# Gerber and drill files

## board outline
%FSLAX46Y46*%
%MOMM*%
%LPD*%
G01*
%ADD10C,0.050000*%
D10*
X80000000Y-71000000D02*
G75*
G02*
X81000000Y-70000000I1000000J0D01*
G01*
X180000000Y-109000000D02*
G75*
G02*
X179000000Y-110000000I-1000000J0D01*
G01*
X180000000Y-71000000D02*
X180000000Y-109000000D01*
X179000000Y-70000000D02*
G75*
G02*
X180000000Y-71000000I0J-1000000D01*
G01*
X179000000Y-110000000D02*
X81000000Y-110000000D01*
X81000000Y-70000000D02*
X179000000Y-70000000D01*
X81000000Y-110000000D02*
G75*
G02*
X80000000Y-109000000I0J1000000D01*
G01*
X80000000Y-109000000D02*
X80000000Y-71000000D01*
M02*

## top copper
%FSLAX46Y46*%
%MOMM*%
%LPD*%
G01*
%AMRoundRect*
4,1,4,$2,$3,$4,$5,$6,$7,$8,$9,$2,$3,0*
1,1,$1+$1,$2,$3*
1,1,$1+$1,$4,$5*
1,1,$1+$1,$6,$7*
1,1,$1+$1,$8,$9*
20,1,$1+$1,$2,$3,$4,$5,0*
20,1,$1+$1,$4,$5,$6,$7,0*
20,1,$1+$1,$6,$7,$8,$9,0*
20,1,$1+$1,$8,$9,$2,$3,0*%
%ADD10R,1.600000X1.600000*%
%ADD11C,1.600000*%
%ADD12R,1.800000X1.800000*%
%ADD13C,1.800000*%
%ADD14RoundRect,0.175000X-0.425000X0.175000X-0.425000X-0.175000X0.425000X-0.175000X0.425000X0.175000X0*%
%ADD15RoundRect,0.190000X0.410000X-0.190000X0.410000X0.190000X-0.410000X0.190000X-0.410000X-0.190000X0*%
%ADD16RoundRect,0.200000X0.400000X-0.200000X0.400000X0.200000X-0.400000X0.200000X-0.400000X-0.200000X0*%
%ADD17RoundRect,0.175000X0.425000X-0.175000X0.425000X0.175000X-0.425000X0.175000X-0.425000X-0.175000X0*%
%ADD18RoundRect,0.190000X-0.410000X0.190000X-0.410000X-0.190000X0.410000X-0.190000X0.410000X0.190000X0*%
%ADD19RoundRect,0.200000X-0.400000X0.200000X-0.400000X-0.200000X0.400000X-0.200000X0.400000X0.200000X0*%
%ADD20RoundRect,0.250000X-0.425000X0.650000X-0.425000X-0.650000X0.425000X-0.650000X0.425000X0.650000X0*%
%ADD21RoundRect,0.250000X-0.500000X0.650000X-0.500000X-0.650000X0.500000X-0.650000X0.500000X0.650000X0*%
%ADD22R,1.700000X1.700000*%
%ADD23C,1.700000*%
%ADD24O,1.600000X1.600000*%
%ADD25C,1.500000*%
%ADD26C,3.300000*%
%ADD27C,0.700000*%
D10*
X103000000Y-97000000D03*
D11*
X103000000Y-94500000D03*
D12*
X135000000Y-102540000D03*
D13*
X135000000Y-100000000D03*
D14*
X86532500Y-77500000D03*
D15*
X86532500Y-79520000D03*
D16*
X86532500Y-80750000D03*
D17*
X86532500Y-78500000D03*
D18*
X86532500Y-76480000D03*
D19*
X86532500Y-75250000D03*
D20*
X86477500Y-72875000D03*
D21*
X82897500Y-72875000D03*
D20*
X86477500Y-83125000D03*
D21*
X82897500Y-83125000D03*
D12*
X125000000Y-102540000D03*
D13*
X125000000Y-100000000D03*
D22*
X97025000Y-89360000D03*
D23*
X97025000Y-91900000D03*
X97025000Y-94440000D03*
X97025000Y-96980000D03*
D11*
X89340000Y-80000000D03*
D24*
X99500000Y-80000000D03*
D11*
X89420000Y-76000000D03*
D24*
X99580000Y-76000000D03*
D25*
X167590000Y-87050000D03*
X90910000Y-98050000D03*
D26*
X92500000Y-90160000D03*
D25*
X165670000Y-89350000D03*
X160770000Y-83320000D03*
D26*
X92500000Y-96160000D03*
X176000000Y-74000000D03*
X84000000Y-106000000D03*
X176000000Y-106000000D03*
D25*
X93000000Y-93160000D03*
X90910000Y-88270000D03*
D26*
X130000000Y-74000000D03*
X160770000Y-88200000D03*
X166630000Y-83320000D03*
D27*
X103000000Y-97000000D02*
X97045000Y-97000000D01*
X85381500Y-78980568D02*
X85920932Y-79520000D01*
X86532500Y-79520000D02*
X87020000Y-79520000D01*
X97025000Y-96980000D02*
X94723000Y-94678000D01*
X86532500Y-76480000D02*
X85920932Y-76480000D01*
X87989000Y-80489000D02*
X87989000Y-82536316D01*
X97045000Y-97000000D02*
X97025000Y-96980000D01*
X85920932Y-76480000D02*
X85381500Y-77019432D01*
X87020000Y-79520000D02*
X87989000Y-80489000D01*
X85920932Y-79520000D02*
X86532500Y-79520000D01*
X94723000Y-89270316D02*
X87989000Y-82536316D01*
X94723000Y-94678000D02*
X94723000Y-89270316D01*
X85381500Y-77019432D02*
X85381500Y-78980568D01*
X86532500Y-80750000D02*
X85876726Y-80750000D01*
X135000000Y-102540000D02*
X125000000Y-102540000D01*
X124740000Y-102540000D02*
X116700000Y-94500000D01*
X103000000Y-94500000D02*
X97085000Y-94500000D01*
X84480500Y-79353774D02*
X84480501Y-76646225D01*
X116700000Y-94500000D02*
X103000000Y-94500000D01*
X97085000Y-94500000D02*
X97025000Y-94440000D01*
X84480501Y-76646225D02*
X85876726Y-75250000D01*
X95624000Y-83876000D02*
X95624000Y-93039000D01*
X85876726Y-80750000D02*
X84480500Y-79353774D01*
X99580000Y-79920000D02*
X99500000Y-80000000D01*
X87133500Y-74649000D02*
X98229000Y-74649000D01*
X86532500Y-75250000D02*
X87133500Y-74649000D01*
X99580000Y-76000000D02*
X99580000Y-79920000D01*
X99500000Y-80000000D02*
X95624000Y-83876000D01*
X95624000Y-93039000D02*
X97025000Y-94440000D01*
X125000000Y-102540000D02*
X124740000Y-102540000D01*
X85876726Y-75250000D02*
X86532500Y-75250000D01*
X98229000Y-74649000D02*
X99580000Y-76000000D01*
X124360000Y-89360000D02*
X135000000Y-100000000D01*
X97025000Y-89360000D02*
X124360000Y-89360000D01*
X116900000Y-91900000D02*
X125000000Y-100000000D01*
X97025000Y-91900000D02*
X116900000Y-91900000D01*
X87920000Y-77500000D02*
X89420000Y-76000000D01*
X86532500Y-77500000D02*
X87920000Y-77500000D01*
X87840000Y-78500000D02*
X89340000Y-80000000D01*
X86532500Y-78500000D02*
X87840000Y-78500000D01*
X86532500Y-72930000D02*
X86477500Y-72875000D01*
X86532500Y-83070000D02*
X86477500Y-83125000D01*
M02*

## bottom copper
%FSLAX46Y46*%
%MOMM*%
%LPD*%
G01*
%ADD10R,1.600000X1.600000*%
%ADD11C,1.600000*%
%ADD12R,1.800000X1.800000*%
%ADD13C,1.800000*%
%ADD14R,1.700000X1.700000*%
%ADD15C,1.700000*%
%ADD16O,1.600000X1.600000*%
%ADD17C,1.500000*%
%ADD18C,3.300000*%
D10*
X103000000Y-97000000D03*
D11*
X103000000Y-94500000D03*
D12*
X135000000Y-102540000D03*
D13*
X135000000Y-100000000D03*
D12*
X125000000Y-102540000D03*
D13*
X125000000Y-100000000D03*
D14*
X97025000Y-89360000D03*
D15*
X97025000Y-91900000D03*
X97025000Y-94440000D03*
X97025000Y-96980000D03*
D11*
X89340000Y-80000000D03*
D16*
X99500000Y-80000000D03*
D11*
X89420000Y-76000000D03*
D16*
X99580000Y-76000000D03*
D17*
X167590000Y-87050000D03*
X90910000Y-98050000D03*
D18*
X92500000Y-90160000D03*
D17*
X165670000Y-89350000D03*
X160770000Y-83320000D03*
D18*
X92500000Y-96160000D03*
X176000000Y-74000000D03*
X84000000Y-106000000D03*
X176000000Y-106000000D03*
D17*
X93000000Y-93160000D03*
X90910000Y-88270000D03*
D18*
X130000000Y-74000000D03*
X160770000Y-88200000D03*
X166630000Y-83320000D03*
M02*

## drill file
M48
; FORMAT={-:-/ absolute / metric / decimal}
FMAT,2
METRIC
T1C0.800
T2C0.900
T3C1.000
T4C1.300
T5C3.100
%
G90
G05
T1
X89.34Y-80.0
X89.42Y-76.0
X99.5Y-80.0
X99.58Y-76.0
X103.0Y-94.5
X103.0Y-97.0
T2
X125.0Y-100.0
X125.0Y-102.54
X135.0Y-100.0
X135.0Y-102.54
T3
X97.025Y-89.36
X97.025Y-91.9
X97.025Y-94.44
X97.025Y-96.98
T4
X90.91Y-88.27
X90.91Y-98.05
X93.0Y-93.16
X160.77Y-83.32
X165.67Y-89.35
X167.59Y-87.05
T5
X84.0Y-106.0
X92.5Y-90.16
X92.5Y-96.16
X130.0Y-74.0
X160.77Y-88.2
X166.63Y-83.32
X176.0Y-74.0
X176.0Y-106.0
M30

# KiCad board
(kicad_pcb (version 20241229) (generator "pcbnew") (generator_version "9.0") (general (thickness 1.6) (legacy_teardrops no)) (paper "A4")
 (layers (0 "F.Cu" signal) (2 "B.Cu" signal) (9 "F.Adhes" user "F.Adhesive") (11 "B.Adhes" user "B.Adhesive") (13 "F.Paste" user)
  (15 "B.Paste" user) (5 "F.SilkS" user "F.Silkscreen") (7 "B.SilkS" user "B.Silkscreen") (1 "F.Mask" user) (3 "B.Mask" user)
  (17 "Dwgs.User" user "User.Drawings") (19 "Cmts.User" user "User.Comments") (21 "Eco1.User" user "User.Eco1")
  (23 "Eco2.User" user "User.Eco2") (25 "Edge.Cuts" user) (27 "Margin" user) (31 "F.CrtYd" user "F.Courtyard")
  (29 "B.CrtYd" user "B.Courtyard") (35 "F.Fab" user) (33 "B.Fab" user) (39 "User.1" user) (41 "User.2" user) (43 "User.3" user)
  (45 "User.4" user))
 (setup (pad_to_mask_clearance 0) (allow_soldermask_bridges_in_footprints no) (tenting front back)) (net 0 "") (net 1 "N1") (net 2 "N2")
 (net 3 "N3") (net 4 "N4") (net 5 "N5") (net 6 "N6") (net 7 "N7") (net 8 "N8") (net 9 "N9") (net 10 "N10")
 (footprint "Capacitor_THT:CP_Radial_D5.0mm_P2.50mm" (layer "F.Cu") (at 103 97 90)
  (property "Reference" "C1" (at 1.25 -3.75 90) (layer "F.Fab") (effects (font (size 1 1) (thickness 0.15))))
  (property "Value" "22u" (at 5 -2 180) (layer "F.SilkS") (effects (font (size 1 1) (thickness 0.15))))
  (pad "1" thru_hole rect (at 0 0 90) (size 1.6 1.6) (drill 0.8) (layers "*.Cu" "*.Mask") (remove_unused_layers no) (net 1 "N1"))
  (pad "2" thru_hole circle (at 2.5 0 90) (size 1.6 1.6) (drill 0.8) (layers "*.Cu" "*.Mask") (remove_unused_layers no) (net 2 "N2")))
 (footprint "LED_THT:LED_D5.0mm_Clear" (layer "F.Cu") (at 135 102.54 90)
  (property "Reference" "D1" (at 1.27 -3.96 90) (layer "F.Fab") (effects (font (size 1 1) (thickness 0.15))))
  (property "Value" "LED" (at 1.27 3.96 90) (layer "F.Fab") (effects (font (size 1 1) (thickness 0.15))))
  (pad "1" thru_hole rect (at 0 0 90) (size 1.8 1.8) (drill 0.9) (layers "*.Cu" "*.Mask") (remove_unused_layers no) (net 2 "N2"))
  (pad "2" thru_hole circle (at 2.54 0 90) (size 1.8 1.8) (drill 0.9) (layers "*.Cu" "*.Mask") (remove_unused_layers no) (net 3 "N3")))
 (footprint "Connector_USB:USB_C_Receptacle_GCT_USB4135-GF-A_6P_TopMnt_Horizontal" (layer "F.Cu") (at 83.5 78 -90)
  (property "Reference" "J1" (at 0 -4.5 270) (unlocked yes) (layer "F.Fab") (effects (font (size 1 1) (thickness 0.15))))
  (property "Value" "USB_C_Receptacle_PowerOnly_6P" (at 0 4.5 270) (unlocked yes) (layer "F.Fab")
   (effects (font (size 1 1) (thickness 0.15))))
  (pad "A5" smd roundrect (at -0.5 -3.0325 270) (size 0.7 1.2) (layers "F.Cu" "F.Mask" "F.Paste") (roundrect_rratio 0.25) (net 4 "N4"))
  (pad "A9" smd roundrect (at 1.52 -3.0325 90) (size 0.76 1.2) (layers "F.Cu" "F.Mask" "F.Paste") (roundrect_rratio 0.25) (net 1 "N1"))
  (pad "A12" smd roundrect (at 2.75 -3.0325 90) (size 0.8 1.2) (layers "F.Cu" "F.Mask" "F.Paste") (roundrect_rratio 0.25) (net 2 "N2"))
  (pad "B5" smd roundrect (at 0.5 -3.0325 90) (size 0.7 1.2) (layers "F.Cu" "F.Mask" "F.Paste") (roundrect_rratio 0.25) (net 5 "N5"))
  (pad "B9" smd roundrect (at -1.52 -3.0325 270) (size 0.76 1.2) (layers "F.Cu" "F.Mask" "F.Paste") (roundrect_rratio 0.25) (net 1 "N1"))
  (pad "B12" smd roundrect (at -2.75 -3.0325 270) (size 0.8 1.2) (layers "F.Cu" "F.Mask" "F.Paste") (roundrect_rratio 0.25) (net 2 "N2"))
  (pad "S1" smd roundrect (at -5.125 -2.9775 270) (size 1.8 1.35) (layers "F.Cu" "F.Mask" "F.Paste") (roundrect_rratio 0.1851851852)
   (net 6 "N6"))
  (pad "S1" smd roundrect (at -5.125 0.6025 270) (size 1.8 1.5) (layers "F.Cu" "F.Mask" "F.Paste") (roundrect_rratio 0.1666666667)
   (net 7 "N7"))
  (pad "S1" smd roundrect (at 5.125 -2.9775 270) (size 1.8 1.35) (layers "F.Cu" "F.Mask" "F.Paste") (roundrect_rratio 0.1851851852)
   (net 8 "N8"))
  (pad "S1" smd roundrect (at 5.125 0.6025 270) (size 1.8 1.5) (layers "F.Cu" "F.Mask" "F.Paste") (roundrect_rratio 0.1666666667)
   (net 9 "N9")))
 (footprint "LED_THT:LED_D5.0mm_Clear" (layer "F.Cu") (at 125 102.54 90)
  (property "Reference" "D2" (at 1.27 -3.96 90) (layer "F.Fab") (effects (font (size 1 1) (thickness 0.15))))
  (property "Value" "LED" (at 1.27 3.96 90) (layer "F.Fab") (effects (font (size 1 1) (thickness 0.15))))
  (pad "1" thru_hole rect (at 0 0 90) (size 1.8 1.8) (drill 0.9) (layers "*.Cu" "*.Mask") (remove_unused_layers no) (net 2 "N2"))
  (pad "2" thru_hole circle (at 2.54 0 90) (size 1.8 1.8) (drill 0.9) (layers "*.Cu" "*.Mask") (remove_unused_layers no) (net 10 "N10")))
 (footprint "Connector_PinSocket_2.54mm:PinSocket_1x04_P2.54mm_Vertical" (layer "F.Cu") (at 97.025 89.36)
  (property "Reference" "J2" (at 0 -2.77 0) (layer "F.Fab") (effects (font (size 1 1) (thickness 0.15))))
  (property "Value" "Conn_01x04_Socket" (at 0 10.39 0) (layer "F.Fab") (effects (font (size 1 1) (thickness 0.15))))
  (pad "1" thru_hole rect (at 0 0) (size 1.7 1.7) (drill 1) (layers "*.Cu" "*.Mask") (remove_unused_layers no) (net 3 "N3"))
  (pad "2" thru_hole circle (at 0 2.54) (size 1.7 1.7) (drill 1) (layers "*.Cu" "*.Mask") (remove_unused_layers no) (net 10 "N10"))
  (pad "3" thru_hole circle (at 0 5.08) (size 1.7 1.7) (drill 1) (layers "*.Cu" "*.Mask") (remove_unused_layers no) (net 2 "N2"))
  (pad "4" thru_hole circle (at 0 7.62) (size 1.7 1.7) (drill 1) (layers "*.Cu" "*.Mask") (remove_unused_layers no) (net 1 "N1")))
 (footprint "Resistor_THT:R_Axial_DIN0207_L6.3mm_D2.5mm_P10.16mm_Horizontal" (layer "F.Cu") (at 89.34 80)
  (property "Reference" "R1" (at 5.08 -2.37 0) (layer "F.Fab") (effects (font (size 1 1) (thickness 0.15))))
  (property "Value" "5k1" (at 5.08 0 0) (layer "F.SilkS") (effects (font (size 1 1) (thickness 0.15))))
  (pad "1" thru_hole circle (at 0 0) (size 1.6 1.6) (drill 0.8) (layers "*.Cu" "*.Mask") (remove_unused_layers no) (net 5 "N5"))
  (pad "2" thru_hole oval (at 10.16 0) (size 1.6 1.6) (drill 0.8) (layers "*.Cu" "*.Mask") (remove_unused_layers no) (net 2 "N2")))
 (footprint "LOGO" (layer "F.Cu") (at 176 90 90)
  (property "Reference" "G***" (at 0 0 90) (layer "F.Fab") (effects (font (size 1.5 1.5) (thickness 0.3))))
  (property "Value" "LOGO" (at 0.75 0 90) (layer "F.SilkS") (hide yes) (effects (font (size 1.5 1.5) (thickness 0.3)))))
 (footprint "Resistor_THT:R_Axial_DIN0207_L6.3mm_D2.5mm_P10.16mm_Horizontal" (layer "F.Cu") (at 89.42 76)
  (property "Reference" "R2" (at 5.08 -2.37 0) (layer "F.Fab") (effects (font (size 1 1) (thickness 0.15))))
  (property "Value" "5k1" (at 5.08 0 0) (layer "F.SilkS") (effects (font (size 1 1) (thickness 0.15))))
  (pad "1" thru_hole circle (at 0 0) (size 1.6 1.6) (drill 0.8) (layers "*.Cu" "*.Mask") (remove_unused_layers no) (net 4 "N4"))
  (pad "2" thru_hole oval (at 10.16 0) (size 1.6 1.6) (drill 0.8) (layers "*.Cu" "*.Mask") (remove_unused_layers no) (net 2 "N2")))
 (gr_arc (start 80 71) (mid 80.292893 70.292893) (end 81 70) (stroke (width 0.05) (type default)) (layer "Edge.Cuts"))
 (gr_arc (start 180 109) (mid 179.707107 109.707107) (end 179 110) (stroke (width 0.05) (type default)) (layer "Edge.Cuts"))
 (gr_line (start 180 71) (end 180 109) (stroke (width 0.05) (type default)) (layer "Edge.Cuts"))
 (gr_arc (start 179 70) (mid 179.707107 70.292893) (end 180 71) (stroke (width 0.05) (type default)) (layer "Edge.Cuts"))
 (gr_line (start 179 110) (end 81 110) (stroke (width 0.05) (type default)) (layer "Edge.Cuts"))
 (gr_line (start 81 70) (end 179 70) (stroke (width 0.05) (type default)) (layer "Edge.Cuts"))
 (gr_arc (start 81 110) (mid 80.292893 109.707107) (end 80 109) (stroke (width 0.05) (type default)) (layer "Edge.Cuts"))
 (gr_line (start 80 109) (end 80 71) (stroke (width 0.05) (type default)) (layer "Edge.Cuts"))
 (via (at 167.59 87.05) (size 1.5) (drill 1.3) (layers "F.Cu" "B.Cu") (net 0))
 (via (at 90.91 98.05) (size 1.5) (drill 1.3) (layers "F.Cu" "B.Cu") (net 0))
 (via (at 92.5 90.16) (size 3.3) (drill 3.1) (layers "F.Cu" "B.Cu") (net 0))
 (via (at 165.67 89.35) (size 1.5) (drill 1.3) (layers "F.Cu" "B.Cu") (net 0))
 (via (at 160.77 83.32) (size 1.5) (drill 1.3) (layers "F.Cu" "B.Cu") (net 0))
 (via (at 92.5 96.16) (size 3.3) (drill 3.1) (layers "F.Cu" "B.Cu") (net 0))
 (via (at 176 74) (size 3.3) (drill 3.1) (layers "F.Cu" "B.Cu") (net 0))
 (via (at 84 106) (size 3.3) (drill 3.1) (layers "F.Cu" "B.Cu") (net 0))
 (via (at 176 106) (size 3.3) (drill 3.1) (layers "F.Cu" "B.Cu") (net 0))
 (via (at 93 93.16) (size 1.5) (drill 1.3) (layers "F.Cu" "B.Cu") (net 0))
 (via (at 90.91 88.27) (size 1.5) (drill 1.3) (layers "F.Cu" "B.Cu") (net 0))
 (via (at 130 74) (size 3.3) (drill 3.1) (layers "F.Cu" "B.Cu") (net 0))
 (via (at 160.77 88.2) (size 3.3) (drill 3.1) (layers "F.Cu" "B.Cu") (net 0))
 (via (at 166.63 83.32) (size 3.3) (drill 3.1) (layers "F.Cu" "B.Cu") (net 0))
 (segment (start 103 97) (end 97.045 97) (width 0.7) (layer "F.Cu") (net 1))
 (segment (start 85.3815 78.980568) (end 85.920932 79.52) (width 0.7) (layer "F.Cu") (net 1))
 (segment (start 86.5325 79.52) (end 87.02 79.52) (width 0.7) (layer "F.Cu") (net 1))
 (segment (start 97.025 96.98) (end 94.723 94.678) (width 0.7) (layer "F.Cu") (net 1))
 (segment (start 86.5325 76.48) (end 85.920932 76.48) (width 0.7) (layer "F.Cu") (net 1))
 (segment (start 87.989 80.489) (end 87.989 82.536316) (width 0.7) (layer "F.Cu") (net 1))
 (segment (start 97.045 97) (end 97.025 96.98) (width 0.7) (layer "F.Cu") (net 1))
 (segment (start 85.920932 76.48) (end 85.3815 77.019432) (width 0.7) (layer "F.Cu") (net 1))
 (segment (start 87.02 79.52) (end 87.989 80.489) (width 0.7) (layer "F.Cu") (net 1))
 (segment (start 85.920932 79.52) (end 86.5325 79.52) (width 0.7) (layer "F.Cu") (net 1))
 (segment (start 94.723 89.270316) (end 87.989 82.536316) (width 0.7) (layer "F.Cu") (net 1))
 (segment (start 94.723 94.678) (end 94.723 89.270316) (width 0.7) (layer "F.Cu") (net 1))
 (segment (start 85.3815 77.019432) (end 85.3815 78.980568) (width 0.7) (layer "F.Cu") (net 1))
 (segment (start 86.5325 80.75) (end 85.876726 80.75) (width 0.7) (layer "F.Cu") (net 2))
 (segment (start 135 102.54) (end 125 102.54) (width 0.7) (layer "F.Cu") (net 2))
 (segment (start 124.74 102.54) (end 116.7 94.5) (width 0.7) (layer "F.Cu") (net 2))
 (segment (start 103 94.5) (end 97.085 94.5) (width 0.7) (layer "F.Cu") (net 2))
 (segment (start 84.4805 79.353774) (end 84.480501 76.646225) (width 0.7) (layer "F.Cu") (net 2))
 (segment (start 116.7 94.5) (end 103 94.5) (width 0.7) (layer "F.Cu") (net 2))
 (segment (start 97.085 94.5) (end 97.025 94.44) (width 0.7) (layer "F.Cu") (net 2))
 (segment (start 84.480501 76.646225) (end 85.876726 75.25) (width 0.7) (layer "F.Cu") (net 2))
 (segment (start 95.624 83.876) (end 95.624 93.039) (width 0.7) (layer "F.Cu") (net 2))
 (segment (start 85.876726 80.75) (end 84.4805 79.353774) (width 0.7) (layer "F.Cu") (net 2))
 (segment (start 99.58 79.92) (end 99.5 80) (width 0.7) (layer "F.Cu") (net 2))
 (segment (start 87.1335 74.649) (end 98.229 74.649) (width 0.7) (layer "F.Cu") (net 2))
 (segment (start 86.5325 75.25) (end 87.1335 74.649) (width 0.7) (layer "F.Cu") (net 2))
 (segment (start 99.58 76) (end 99.58 79.92) (width 0.7) (layer "F.Cu") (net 2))
 (segment (start 99.5 80) (end 95.624 83.876) (width 0.7) (layer "F.Cu") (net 2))
 (segment (start 95.624 93.039) (end 97.025 94.44) (width 0.7) (layer "F.Cu") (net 2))
 (segment (start 125 102.54) (end 124.74 102.54) (width 0.7) (layer "F.Cu") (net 2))
 (segment (start 85.876726 75.25) (end 86.5325 75.25) (width 0.7) (layer "F.Cu") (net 2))
 (segment (start 98.229 74.649) (end 99.58 76) (width 0.7) (layer "F.Cu") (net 2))
 (segment (start 124.36 89.36) (end 135 100) (width 0.7) (layer "F.Cu") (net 3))
 (segment (start 97.025 89.36) (end 124.36 89.36) (width 0.7) (layer "F.Cu") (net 3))
 (segment (start 116.9 91.9) (end 125 100) (width 0.7) (layer "F.Cu") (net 10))
 (segment (start 97.025 91.9) (end 116.9 91.9) (width 0.7) (layer "F.Cu") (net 10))
 (segment (start 87.92 77.5) (end 89.42 76) (width 0.7) (layer "F.Cu") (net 4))
 (segment (start 86.5325 77.5) (end 87.92 77.5) (width 0.7) (layer "F.Cu") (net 4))
 (segment (start 87.84 78.5) (end 89.34 80) (width 0.7) (layer "F.Cu") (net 5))
 (segment (start 86.5325 78.5) (end 87.84 78.5) (width 0.7) (layer "F.Cu") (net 5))
 (segment (start 86.5325 72.93) (end 86.4775 72.875) (width 0.7) (layer "F.Cu") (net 6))
 (segment (start 86.5325 83.07) (end 86.4775 83.125) (width 0.7) (layer "F.Cu") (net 8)))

